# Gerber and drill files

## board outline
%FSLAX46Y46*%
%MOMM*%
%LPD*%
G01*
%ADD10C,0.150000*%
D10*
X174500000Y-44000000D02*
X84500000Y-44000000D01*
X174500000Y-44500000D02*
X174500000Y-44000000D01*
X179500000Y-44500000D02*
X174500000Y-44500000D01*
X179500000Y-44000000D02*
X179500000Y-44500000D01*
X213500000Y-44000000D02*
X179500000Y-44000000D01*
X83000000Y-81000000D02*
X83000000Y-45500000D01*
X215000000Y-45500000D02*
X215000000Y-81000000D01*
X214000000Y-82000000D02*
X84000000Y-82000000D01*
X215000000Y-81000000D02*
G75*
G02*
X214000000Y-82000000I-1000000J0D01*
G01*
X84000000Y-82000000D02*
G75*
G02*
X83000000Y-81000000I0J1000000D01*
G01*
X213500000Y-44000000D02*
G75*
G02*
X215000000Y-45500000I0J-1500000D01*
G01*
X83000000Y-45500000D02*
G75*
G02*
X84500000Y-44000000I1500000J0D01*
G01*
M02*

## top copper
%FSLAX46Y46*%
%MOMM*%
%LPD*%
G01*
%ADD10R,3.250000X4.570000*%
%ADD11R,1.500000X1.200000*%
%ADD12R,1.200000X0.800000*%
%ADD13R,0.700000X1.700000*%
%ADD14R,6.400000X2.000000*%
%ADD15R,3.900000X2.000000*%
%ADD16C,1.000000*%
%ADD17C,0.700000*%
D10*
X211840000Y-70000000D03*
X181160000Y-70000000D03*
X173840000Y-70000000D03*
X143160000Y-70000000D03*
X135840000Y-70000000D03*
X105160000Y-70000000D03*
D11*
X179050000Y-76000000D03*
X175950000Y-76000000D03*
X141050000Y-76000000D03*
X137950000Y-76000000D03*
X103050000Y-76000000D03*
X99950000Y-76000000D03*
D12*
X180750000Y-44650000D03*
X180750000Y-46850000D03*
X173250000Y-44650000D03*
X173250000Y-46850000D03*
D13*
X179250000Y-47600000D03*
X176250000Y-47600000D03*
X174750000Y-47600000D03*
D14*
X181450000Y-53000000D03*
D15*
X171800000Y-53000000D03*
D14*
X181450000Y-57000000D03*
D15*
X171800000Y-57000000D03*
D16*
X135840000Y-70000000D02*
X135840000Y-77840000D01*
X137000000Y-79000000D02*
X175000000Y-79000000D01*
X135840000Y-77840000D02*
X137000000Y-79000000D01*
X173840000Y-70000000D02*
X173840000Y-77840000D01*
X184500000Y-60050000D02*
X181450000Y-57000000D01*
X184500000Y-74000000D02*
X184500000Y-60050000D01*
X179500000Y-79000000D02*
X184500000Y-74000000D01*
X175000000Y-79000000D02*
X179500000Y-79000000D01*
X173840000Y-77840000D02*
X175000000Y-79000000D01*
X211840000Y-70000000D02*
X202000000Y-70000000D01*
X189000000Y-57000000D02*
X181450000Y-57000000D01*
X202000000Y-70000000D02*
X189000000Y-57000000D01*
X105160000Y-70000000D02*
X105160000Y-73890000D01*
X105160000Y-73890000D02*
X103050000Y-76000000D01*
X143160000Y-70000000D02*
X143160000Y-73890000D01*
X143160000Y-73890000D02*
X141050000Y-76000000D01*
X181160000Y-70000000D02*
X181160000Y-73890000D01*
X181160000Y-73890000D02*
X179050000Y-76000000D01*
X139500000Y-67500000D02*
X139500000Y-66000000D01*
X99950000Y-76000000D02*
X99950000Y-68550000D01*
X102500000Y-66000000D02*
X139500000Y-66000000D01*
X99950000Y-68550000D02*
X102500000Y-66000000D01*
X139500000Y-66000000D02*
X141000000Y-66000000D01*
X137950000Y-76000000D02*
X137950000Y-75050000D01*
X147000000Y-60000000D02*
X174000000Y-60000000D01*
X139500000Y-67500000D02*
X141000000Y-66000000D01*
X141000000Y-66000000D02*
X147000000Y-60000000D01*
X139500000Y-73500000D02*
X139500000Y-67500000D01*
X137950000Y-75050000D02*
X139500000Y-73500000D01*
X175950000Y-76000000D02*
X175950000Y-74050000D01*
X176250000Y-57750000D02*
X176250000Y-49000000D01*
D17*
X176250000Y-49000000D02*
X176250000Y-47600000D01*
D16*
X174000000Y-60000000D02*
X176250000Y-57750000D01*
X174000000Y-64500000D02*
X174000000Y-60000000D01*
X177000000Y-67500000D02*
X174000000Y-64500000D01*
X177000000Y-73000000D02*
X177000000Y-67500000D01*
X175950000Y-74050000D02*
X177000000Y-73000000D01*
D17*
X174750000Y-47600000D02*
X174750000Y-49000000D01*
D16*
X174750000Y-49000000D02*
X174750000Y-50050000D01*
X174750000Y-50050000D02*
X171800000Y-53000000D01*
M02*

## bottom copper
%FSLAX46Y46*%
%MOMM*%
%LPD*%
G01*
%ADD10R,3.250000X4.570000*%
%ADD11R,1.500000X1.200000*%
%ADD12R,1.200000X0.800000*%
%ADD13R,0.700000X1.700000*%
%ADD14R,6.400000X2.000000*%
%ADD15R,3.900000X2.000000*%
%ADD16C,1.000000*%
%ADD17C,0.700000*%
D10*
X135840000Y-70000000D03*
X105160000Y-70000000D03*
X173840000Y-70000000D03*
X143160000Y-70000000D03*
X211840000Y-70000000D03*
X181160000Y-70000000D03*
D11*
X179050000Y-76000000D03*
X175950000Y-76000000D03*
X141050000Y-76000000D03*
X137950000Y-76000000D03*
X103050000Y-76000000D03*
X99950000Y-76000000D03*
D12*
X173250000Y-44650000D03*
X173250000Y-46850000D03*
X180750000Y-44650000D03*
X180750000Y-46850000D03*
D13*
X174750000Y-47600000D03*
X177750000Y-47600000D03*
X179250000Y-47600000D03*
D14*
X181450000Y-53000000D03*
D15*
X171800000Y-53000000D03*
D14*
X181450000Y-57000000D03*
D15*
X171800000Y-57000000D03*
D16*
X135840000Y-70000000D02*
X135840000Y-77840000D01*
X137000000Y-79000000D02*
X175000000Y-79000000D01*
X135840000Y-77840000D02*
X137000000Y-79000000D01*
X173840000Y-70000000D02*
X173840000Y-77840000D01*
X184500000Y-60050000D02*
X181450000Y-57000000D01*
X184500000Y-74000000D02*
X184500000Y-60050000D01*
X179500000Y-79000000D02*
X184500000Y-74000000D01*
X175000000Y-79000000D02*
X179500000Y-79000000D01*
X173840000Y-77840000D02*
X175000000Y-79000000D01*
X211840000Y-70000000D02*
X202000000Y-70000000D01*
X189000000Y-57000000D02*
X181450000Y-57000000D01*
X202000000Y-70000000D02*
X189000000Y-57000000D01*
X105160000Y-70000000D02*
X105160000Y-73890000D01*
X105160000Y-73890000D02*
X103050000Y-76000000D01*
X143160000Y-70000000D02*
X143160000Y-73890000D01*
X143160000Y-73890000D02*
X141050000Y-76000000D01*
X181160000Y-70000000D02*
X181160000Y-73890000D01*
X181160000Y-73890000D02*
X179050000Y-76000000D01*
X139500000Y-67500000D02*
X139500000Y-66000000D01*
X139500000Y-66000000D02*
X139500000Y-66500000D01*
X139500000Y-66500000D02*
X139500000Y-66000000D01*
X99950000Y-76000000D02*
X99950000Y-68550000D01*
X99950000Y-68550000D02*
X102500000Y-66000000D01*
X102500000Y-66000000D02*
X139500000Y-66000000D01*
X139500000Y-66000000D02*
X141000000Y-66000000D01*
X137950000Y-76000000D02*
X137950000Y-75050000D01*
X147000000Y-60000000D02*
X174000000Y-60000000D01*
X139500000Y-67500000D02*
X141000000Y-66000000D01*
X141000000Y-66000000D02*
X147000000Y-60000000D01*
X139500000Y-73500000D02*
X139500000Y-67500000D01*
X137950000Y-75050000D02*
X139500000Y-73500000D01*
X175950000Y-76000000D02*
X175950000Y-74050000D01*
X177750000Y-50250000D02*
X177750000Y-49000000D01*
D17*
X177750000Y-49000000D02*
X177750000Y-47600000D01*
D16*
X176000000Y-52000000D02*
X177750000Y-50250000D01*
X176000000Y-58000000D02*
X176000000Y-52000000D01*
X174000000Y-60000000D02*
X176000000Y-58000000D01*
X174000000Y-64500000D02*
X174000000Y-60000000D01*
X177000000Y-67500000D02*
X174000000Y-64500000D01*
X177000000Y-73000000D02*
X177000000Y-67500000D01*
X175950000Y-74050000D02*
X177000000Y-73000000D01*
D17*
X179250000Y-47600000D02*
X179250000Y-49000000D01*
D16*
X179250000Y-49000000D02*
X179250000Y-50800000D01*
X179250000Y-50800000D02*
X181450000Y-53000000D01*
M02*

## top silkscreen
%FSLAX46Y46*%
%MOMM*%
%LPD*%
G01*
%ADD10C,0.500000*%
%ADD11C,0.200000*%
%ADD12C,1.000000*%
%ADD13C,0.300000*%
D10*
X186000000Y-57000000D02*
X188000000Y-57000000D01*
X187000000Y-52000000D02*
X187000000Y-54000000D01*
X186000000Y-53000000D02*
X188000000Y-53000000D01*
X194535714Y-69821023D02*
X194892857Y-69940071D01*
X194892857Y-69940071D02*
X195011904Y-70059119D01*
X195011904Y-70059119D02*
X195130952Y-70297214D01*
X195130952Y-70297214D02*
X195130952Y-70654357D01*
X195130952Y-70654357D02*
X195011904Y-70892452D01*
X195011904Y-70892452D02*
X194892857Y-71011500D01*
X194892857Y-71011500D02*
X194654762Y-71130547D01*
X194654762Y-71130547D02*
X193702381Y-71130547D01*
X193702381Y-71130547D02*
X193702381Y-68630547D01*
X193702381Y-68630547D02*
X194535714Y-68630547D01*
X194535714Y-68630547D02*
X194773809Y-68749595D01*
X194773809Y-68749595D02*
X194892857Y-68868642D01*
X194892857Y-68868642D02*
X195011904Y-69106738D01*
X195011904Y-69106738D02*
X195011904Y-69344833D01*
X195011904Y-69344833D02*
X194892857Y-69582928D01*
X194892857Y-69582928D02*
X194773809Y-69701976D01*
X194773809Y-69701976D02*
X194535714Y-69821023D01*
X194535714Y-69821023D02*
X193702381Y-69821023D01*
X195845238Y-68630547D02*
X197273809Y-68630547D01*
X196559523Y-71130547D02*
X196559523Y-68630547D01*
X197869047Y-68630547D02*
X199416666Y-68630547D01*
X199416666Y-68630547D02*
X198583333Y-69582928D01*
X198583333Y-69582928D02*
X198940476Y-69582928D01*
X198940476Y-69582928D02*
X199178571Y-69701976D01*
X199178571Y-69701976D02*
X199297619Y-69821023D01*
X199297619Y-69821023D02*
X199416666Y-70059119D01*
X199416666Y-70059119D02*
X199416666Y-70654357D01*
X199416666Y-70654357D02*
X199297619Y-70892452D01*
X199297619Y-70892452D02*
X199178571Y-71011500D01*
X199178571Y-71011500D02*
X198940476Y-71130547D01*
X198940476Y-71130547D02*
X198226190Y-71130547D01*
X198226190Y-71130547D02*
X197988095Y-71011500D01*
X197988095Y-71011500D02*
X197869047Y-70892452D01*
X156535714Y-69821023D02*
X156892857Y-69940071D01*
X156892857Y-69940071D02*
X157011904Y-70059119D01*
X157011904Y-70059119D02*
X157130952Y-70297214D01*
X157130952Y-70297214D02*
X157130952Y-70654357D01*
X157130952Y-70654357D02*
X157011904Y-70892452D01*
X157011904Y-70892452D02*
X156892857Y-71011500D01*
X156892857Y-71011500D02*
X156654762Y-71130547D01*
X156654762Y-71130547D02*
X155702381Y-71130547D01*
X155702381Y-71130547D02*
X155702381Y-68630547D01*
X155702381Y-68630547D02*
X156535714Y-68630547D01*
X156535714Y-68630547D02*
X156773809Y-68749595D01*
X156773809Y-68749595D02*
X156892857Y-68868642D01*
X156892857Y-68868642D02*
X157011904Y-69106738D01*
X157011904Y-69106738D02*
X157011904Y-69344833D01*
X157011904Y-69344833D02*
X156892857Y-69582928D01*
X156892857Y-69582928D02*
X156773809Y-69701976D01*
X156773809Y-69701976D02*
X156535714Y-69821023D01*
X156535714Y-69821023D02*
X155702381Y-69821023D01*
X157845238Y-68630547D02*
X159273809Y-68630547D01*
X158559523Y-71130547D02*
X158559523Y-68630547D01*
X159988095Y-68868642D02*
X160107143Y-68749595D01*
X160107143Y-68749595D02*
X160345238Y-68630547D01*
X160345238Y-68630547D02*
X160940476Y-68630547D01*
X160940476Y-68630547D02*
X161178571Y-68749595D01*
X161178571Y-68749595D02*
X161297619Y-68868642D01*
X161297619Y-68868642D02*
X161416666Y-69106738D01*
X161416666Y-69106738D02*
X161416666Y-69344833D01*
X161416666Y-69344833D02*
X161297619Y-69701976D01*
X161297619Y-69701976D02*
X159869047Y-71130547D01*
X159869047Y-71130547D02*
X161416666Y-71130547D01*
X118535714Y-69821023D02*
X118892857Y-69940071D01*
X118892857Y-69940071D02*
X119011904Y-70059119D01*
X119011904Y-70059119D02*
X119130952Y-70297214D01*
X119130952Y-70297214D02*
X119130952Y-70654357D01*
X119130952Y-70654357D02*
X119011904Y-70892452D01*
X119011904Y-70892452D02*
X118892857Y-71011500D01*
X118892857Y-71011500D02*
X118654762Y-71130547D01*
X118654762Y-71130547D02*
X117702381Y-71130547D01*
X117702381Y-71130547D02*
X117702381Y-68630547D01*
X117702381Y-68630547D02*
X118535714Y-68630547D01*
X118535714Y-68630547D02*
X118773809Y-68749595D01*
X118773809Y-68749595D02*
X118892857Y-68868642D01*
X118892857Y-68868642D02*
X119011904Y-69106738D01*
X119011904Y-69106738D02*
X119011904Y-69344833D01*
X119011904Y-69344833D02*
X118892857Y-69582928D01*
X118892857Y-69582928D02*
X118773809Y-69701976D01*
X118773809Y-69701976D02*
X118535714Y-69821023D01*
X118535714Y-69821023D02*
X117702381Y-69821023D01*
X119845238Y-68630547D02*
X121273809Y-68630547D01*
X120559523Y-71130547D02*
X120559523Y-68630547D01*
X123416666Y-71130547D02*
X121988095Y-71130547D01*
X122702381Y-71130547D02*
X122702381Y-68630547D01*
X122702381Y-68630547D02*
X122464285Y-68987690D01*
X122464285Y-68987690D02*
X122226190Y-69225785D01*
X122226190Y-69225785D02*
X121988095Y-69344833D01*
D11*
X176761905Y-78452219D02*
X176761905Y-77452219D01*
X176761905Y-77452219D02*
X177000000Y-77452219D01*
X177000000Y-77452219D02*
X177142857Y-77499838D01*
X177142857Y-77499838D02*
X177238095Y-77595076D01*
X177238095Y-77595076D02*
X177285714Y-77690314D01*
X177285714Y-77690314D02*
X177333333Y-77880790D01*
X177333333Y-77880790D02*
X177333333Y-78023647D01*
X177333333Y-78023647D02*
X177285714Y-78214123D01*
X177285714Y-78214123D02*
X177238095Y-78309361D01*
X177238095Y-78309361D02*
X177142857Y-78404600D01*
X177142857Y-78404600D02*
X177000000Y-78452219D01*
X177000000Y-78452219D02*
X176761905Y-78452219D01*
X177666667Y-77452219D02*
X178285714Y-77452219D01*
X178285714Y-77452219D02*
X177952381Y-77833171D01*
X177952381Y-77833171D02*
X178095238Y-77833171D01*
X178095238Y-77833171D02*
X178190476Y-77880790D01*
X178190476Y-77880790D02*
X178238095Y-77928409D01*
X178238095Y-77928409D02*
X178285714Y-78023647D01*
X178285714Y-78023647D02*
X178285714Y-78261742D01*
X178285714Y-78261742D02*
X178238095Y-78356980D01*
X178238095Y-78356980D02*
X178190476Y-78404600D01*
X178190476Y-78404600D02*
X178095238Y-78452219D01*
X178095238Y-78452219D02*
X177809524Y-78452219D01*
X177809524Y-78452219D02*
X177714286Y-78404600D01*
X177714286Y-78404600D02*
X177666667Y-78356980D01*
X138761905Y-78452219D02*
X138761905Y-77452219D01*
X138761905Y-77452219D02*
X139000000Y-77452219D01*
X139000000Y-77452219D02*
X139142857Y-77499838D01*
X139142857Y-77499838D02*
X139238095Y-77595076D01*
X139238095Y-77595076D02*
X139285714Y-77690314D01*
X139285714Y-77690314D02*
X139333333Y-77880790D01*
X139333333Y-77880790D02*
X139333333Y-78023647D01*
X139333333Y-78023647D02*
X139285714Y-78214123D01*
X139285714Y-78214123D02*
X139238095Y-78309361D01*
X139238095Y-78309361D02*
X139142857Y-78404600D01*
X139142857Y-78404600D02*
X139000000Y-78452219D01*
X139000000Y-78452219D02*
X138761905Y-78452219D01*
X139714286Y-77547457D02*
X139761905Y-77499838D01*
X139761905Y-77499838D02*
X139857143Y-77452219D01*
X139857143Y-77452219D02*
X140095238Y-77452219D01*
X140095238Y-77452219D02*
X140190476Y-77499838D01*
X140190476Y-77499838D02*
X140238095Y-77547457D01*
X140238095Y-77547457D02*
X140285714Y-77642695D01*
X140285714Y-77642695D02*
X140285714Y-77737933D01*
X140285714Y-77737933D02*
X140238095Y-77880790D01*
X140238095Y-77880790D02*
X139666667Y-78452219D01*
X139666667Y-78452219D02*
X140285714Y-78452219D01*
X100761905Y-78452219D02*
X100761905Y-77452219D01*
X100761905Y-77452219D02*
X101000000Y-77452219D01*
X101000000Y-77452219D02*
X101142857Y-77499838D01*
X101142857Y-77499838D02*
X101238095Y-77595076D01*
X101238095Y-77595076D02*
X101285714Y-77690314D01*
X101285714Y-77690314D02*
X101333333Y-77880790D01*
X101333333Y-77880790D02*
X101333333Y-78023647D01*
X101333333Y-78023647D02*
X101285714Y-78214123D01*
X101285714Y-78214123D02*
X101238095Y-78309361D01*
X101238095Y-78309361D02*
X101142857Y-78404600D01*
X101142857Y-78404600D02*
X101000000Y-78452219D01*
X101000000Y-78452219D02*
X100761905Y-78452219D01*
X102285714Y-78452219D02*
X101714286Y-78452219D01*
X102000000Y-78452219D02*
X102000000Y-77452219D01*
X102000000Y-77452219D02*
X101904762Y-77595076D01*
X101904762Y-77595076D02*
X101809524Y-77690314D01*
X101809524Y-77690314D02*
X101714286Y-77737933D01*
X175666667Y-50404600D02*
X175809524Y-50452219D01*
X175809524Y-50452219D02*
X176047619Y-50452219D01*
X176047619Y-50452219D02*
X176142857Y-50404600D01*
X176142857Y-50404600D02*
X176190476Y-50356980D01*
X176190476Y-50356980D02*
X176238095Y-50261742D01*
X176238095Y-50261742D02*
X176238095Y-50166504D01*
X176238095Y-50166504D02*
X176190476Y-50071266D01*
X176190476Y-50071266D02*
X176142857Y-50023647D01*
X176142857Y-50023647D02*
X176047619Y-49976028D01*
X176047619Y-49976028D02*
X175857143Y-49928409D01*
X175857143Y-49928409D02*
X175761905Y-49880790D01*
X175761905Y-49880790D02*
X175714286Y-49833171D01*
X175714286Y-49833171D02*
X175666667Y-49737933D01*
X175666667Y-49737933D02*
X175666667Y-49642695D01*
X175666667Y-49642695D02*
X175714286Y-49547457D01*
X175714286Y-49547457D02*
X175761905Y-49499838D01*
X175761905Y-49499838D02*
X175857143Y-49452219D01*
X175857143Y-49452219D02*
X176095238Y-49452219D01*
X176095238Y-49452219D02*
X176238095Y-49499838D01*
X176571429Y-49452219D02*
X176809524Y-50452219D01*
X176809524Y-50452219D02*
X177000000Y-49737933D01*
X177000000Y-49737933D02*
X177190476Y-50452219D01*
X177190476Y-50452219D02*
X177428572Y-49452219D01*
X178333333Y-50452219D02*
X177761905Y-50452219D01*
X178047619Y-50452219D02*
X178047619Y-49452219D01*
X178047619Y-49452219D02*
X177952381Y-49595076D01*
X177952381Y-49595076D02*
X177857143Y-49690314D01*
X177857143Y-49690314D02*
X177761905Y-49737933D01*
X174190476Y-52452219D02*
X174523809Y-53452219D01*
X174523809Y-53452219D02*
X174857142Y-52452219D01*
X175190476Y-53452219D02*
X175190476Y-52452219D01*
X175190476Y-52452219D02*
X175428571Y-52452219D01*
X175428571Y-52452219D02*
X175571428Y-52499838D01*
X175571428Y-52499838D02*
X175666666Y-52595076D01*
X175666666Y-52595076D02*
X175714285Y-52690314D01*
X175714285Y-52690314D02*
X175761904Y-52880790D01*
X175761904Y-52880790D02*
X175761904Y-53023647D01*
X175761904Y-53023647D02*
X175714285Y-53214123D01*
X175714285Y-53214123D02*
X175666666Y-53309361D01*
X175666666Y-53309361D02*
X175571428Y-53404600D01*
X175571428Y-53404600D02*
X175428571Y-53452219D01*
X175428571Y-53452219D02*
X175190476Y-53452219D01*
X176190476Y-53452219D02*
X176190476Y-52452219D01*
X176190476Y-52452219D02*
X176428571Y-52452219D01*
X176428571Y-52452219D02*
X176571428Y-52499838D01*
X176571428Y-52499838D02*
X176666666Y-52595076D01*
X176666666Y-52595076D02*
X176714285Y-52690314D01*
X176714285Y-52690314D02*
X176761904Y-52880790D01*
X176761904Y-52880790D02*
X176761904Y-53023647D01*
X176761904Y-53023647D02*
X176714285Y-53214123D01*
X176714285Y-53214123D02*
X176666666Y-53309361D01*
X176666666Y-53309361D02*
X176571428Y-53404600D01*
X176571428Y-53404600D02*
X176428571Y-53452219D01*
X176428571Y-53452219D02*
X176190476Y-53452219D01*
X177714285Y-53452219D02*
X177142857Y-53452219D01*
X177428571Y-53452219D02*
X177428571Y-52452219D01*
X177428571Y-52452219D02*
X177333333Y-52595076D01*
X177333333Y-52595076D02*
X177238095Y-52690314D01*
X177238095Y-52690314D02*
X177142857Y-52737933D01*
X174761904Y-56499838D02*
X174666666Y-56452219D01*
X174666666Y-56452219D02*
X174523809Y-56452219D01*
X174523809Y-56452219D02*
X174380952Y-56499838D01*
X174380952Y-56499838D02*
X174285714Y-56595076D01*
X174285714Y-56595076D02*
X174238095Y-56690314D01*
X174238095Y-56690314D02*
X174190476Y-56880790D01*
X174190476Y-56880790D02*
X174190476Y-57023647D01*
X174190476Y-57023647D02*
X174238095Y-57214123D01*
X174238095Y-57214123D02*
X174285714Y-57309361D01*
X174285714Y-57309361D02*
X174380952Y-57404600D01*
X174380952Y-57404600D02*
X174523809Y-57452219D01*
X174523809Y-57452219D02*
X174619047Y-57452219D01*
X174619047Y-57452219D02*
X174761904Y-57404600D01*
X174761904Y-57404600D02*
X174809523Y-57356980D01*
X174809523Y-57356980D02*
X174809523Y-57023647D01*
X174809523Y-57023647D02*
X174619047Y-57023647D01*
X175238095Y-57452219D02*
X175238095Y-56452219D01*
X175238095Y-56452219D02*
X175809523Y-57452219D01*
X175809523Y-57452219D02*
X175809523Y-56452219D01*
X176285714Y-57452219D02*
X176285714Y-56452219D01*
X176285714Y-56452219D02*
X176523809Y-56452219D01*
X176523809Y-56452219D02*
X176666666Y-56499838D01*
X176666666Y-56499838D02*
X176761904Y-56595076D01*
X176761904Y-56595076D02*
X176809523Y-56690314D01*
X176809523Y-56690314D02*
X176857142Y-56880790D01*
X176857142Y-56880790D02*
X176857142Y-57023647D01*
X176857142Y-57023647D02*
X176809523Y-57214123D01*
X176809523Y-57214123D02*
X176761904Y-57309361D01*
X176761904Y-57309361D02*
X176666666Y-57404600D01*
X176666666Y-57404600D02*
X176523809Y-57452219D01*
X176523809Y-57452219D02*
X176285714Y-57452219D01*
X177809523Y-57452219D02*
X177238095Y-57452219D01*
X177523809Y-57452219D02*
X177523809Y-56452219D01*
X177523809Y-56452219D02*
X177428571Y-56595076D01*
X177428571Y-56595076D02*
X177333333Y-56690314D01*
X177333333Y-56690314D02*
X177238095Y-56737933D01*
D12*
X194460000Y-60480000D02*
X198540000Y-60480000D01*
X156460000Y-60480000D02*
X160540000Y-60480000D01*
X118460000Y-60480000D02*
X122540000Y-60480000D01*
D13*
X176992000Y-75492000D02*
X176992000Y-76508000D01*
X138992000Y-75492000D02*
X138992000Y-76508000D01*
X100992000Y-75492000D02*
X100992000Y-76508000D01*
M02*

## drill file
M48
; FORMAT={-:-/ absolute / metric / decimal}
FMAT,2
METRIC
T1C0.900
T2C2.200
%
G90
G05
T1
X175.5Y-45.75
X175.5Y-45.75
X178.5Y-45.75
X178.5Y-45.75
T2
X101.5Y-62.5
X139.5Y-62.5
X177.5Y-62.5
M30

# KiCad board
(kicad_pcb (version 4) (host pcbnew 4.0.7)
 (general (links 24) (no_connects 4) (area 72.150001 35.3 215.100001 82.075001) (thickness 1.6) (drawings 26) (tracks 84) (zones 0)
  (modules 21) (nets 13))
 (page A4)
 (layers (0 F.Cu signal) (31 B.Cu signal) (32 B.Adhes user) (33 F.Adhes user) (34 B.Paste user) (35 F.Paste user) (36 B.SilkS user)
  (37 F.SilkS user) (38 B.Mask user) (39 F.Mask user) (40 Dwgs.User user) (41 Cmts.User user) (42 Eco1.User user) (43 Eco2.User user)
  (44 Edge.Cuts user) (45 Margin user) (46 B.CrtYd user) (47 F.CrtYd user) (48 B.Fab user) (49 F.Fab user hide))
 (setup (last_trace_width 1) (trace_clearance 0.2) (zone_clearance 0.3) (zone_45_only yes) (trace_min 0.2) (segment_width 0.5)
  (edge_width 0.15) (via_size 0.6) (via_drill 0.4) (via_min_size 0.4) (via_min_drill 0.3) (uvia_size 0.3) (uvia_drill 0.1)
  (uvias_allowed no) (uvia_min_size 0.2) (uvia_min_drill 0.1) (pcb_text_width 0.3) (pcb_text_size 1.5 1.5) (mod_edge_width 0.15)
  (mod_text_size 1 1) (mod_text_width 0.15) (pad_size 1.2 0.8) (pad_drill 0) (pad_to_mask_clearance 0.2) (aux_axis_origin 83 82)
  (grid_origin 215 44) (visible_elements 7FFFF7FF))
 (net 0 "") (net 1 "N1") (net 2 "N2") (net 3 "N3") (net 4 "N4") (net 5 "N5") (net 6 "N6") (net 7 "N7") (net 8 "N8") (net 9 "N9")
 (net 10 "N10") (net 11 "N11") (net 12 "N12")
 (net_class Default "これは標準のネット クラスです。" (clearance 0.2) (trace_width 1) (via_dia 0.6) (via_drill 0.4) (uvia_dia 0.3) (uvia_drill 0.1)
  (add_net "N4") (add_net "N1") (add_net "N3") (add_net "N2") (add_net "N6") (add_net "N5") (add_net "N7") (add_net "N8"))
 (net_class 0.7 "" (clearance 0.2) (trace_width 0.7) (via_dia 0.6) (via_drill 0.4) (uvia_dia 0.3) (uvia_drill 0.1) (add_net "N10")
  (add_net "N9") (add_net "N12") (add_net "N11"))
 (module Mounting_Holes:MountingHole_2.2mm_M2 (layer F.Cu) (at 101.5 62.5)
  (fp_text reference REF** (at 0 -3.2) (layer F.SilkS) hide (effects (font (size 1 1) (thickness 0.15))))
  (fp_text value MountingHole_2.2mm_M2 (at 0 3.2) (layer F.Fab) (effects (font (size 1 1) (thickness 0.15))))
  (pad 1 np_thru_hole circle (at 0 0) (size 2.2 2.2) (drill 2.2) (layers *.Cu *.Mask)))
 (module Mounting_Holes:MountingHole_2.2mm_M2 (layer F.Cu) (at 139.5 62.5)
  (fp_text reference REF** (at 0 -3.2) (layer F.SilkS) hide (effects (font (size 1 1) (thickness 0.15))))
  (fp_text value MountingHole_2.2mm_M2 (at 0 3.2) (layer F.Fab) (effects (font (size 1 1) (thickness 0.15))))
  (pad 1 np_thru_hole circle (at 0 0) (size 2.2 2.2) (drill 2.2) (layers *.Cu *.Mask)))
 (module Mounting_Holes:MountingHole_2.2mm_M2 (layer F.Cu) (at 177.5 62.5)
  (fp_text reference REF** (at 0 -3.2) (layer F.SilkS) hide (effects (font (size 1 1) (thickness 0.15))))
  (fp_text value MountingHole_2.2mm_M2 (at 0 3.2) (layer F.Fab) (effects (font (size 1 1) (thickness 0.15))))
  (pad 1 np_thru_hole circle (at 0 0) (size 2.2 2.2) (drill 2.2) (layers *.Cu *.Mask)))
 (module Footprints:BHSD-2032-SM (layer F.Cu) (at 196.5 70)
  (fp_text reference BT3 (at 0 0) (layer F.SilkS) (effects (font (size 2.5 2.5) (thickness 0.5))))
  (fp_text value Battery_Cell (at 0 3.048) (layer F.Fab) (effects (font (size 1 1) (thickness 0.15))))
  (fp_line (start -2.04 -9.52) (end 2.04 -9.52) (layer F.SilkS) (width 1))
  (pad 2 smd rect (at 15.34 0) (size 3.25 4.57) (layers F.Cu F.Paste F.Mask) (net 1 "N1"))
  (pad 1 smd rect (at -15.34 0) (size 3.25 4.57) (layers F.Cu F.Paste F.Mask) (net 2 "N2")))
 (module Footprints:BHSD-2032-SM (layer F.Cu) (at 158.5 70)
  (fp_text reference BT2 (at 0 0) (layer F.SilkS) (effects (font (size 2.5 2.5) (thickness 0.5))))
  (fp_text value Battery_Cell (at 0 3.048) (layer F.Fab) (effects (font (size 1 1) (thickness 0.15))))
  (fp_line (start -2.04 -9.52) (end 2.04 -9.52) (layer F.SilkS) (width 1))
  (pad 2 smd rect (at 15.34 0) (size 3.25 4.57) (layers F.Cu F.Paste F.Mask) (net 1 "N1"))
  (pad 1 smd rect (at -15.34 0) (size 3.25 4.57) (layers F.Cu F.Paste F.Mask) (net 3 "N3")))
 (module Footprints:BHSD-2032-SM (layer F.Cu) (at 120.5 70)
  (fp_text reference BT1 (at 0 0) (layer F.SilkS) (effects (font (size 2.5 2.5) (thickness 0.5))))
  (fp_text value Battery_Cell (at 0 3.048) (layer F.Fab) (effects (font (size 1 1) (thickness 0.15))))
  (fp_line (start -2.04 -9.52) (end 2.04 -9.52) (layer F.SilkS) (width 1))
  (pad 2 smd rect (at 15.34 0) (size 3.25 4.57) (layers F.Cu F.Paste F.Mask) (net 1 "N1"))
  (pad 1 smd rect (at -15.34 0) (size 3.25 4.57) (layers F.Cu F.Paste F.Mask) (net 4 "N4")))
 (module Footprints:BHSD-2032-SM (layer B.Cu) (at 120.5 70)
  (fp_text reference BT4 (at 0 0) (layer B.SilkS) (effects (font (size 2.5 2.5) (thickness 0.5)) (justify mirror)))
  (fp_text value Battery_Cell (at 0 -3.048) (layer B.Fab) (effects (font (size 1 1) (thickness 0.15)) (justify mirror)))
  (pad 2 smd rect (at 15.34 0) (size 3.25 4.57) (layers B.Cu B.Paste B.Mask) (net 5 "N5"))
  (pad 1 smd rect (at -15.34 0) (size 3.25 4.57) (layers B.Cu B.Paste B.Mask) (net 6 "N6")))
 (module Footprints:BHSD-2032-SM (layer B.Cu) (at 158.5 70)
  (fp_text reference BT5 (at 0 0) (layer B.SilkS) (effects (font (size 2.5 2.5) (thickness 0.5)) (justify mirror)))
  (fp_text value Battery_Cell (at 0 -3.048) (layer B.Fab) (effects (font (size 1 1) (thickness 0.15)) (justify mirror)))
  (pad 2 smd rect (at 15.34 0) (size 3.25 4.57) (layers B.Cu B.Paste B.Mask) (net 5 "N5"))
  (pad 1 smd rect (at -15.34 0) (size 3.25 4.57) (layers B.Cu B.Paste B.Mask) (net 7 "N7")))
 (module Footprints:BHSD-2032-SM (layer B.Cu) (at 196.5 70)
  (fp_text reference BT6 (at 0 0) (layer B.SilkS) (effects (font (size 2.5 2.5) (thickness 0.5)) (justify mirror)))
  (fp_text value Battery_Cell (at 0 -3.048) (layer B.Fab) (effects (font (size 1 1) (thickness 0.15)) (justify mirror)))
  (pad 2 smd rect (at 15.34 0) (size 3.25 4.57) (layers B.Cu B.Paste B.Mask) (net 5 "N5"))
  (pad 1 smd rect (at -15.34 0) (size 3.25 4.57) (layers B.Cu B.Paste B.Mask) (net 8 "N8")))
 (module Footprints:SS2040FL (layer B.Cu) (at 177.5 76)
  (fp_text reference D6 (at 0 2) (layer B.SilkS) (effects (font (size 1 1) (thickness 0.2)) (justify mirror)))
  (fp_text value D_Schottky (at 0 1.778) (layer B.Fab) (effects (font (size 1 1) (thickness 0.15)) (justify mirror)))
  (pad 2 smd rect (at 1.55 0) (size 1.5 1.2) (layers B.Cu B.Paste B.Mask) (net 8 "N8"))
  (pad 1 smd rect (at -1.55 0) (size 1.5 1.2) (layers B.Cu B.Paste B.Mask) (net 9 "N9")))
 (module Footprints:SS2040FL (layer B.Cu) (at 139.5 76)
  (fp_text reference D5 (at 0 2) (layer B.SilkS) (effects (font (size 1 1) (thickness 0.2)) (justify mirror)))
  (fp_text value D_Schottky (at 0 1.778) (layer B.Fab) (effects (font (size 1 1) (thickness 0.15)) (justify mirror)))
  (pad 2 smd rect (at 1.55 0) (size 1.5 1.2) (layers B.Cu B.Paste B.Mask) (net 7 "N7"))
  (pad 1 smd rect (at -1.55 0) (size 1.5 1.2) (layers B.Cu B.Paste B.Mask) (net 9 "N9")))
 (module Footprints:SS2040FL (layer B.Cu) (at 101.5 76)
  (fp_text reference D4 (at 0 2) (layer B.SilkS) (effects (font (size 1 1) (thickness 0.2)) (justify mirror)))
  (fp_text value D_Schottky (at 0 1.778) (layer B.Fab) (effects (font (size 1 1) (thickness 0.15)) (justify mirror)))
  (pad 2 smd rect (at 1.55 0) (size 1.5 1.2) (layers B.Cu B.Paste B.Mask) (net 6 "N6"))
  (pad 1 smd rect (at -1.55 0) (size 1.5 1.2) (layers B.Cu B.Paste B.Mask) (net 9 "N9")))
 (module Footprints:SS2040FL (layer F.Cu) (at 177.5 76)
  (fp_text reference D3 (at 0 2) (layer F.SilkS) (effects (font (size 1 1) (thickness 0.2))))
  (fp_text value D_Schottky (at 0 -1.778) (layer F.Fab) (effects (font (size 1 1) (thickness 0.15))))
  (fp_line (start -0.508 -0.508) (end -0.508 0.508) (layer F.SilkS) (width 0.3))
  (pad 2 smd rect (at 1.55 0) (size 1.5 1.2) (layers F.Cu F.Paste F.Mask) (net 2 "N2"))
  (pad 1 smd rect (at -1.55 0) (size 1.5 1.2) (layers F.Cu F.Paste F.Mask) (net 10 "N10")))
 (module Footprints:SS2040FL (layer F.Cu) (at 139.5 76)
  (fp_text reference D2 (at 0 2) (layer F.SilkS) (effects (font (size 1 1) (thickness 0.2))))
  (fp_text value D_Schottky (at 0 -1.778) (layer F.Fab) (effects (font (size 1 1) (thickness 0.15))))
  (fp_line (start -0.508 -0.508) (end -0.508 0.508) (layer F.SilkS) (width 0.3))
  (pad 2 smd rect (at 1.55 0) (size 1.5 1.2) (layers F.Cu F.Paste F.Mask) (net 3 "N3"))
  (pad 1 smd rect (at -1.55 0) (size 1.5 1.2) (layers F.Cu F.Paste F.Mask) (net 10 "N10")))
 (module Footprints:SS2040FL (layer F.Cu) (at 101.5 76)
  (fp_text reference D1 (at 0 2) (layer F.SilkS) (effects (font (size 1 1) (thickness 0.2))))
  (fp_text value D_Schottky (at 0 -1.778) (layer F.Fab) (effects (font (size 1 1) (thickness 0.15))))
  (fp_line (start -0.508 -0.508) (end -0.508 0.508) (layer F.SilkS) (width 0.3))
  (pad 2 smd rect (at 1.55 0) (size 1.5 1.2) (layers F.Cu F.Paste F.Mask) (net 4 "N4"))
  (pad 1 smd rect (at -1.55 0) (size 1.5 1.2) (layers F.Cu F.Paste F.Mask) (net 10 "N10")))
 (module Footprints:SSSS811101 (layer B.Cu) (at 177 45.75)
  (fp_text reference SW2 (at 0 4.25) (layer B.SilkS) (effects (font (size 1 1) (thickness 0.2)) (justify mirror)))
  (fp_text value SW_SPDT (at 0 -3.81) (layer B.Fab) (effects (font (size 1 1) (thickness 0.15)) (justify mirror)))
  (pad "" np_thru_hole circle (at -1.5 0) (size 0.9 0.9) (drill 0.9) (layers *.Cu *.Mask))
  (pad "" np_thru_hole circle (at 1.5 0) (size 0.9 0.9) (drill 0.9) (layers *.Cu *.Mask))
  (pad "" smd rect (at -3.75 -1.1) (size 1.2 0.8) (layers B.Cu B.Paste B.Mask))
  (pad "" smd rect (at -3.75 1.1) (size 1.2 0.8) (layers B.Cu B.Paste B.Mask))
  (pad "" smd rect (at 3.75 -1.1) (size 1.2 0.8) (layers B.Cu B.Paste B.Mask))
  (pad "" smd rect (at 3.75 1.1) (size 1.2 0.8) (layers B.Cu B.Paste B.Mask))
  (pad 1 smd rect (at -2.25 1.85) (size 0.7 1.7) (layers B.Cu B.Paste B.Mask))
  (pad 2 smd rect (at 0.75 1.85) (size 0.7 1.7) (layers B.Cu B.Paste B.Mask) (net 9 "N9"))
  (pad 3 smd rect (at 2.25 1.85) (size 0.7 1.7) (layers B.Cu B.Paste B.Mask) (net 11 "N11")))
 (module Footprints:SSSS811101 (layer F.Cu) (at 177 45.75 180)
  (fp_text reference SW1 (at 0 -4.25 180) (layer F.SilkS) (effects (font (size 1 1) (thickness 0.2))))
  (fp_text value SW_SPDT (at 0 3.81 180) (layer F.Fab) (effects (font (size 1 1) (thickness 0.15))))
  (pad "" np_thru_hole circle (at -1.5 0 180) (size 0.9 0.9) (drill 0.9) (layers *.Cu *.Mask))
  (pad "" np_thru_hole circle (at 1.5 0 180) (size 0.9 0.9) (drill 0.9) (layers *.Cu *.Mask))
  (pad "" smd rect (at -3.75 1.1 180) (size 1.2 0.8) (layers F.Cu F.Paste F.Mask))
  (pad "" smd rect (at -3.75 -1.1 180) (size 1.2 0.8) (layers F.Cu F.Paste F.Mask))
  (pad "" smd rect (at 3.75 1.1 180) (size 1.2 0.8) (layers F.Cu F.Paste F.Mask))
  (pad "" smd rect (at 3.75 -1.1 180) (size 1.2 0.8) (layers F.Cu F.Paste F.Mask))
  (pad 1 smd rect (at -2.25 -1.85 180) (size 0.7 1.7) (layers F.Cu F.Paste F.Mask))
  (pad 2 smd rect (at 0.75 -1.85 180) (size 0.7 1.7) (layers F.Cu F.Paste F.Mask) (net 10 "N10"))
  (pad 3 smd rect (at 2.25 -1.85 180) (size 0.7 1.7) (layers F.Cu F.Paste F.Mask) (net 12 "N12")))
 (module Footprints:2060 (layer B.Cu) (at 176 53 180)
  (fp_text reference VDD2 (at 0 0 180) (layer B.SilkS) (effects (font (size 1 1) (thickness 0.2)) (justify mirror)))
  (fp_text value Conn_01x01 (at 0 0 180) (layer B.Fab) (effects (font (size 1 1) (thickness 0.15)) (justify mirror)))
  (pad 1 smd rect (at -5.45 0 180) (size 6.4 2) (layers B.Cu B.Paste B.Mask) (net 11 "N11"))
  (pad 1 smd rect (at 4.2 0 180) (size 3.9 2) (layers B.Cu B.Paste B.Mask) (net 11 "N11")))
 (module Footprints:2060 (layer F.Cu) (at 176 53 180)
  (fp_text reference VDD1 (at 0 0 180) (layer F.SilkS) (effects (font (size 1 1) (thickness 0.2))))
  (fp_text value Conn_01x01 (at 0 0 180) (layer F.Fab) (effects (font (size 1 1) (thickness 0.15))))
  (pad 1 smd rect (at -5.45 0 180) (size 6.4 2) (layers F.Cu F.Paste F.Mask) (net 12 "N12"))
  (pad 1 smd rect (at 4.2 0 180) (size 3.9 2) (layers F.Cu F.Paste F.Mask) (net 12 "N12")))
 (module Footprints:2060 (layer B.Cu) (at 176 57 180)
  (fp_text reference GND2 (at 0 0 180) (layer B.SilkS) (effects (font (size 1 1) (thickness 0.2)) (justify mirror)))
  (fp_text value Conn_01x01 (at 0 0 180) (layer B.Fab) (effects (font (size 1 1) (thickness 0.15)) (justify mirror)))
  (pad 1 smd rect (at -5.45 0 180) (size 6.4 2) (layers B.Cu B.Paste B.Mask) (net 5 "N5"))
  (pad 1 smd rect (at 4.2 0 180) (size 3.9 2) (layers B.Cu B.Paste B.Mask) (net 5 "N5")))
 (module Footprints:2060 (layer F.Cu) (at 176 57 180)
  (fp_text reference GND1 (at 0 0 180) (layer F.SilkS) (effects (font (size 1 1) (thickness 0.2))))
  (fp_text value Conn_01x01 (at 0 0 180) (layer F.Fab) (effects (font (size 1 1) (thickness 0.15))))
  (pad 1 smd rect (at -5.45 0 180) (size 6.4 2) (layers F.Cu F.Paste F.Mask) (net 1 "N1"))
  (pad 1 smd rect (at 4.2 0 180) (size 3.9 2) (layers F.Cu F.Paste F.Mask) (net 1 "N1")))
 (gr_line (start 186 57) (end 188 57) (angle 90) (layer F.SilkS) (width 0.5))
 (gr_line (start 187 52) (end 187 54) (angle 90) (layer F.SilkS) (width 0.5))
 (gr_line (start 186 53) (end 188 53) (angle 90) (layer F.SilkS) (width 0.5))
 (gr_line (start 174.5 44) (end 84.5 44) (angle 90) (layer Edge.Cuts) (width 0.15))
 (gr_line (start 174.5 44.5) (end 174.5 44) (angle 90) (layer Edge.Cuts) (width 0.15))
 (gr_line (start 179.5 44.5) (end 174.5 44.5) (angle 90) (layer Edge.Cuts) (width 0.15))
 (gr_line (start 179.5 44) (end 179.5 44.5) (angle 90) (layer Edge.Cuts) (width 0.15))
 (gr_line (start 213.5 44) (end 179.5 44) (angle 90) (layer Edge.Cuts) (width 0.15))
 (gr_line (start 83 81) (end 83 45.5) (angle 90) (layer Edge.Cuts) (width 0.15))
 (gr_line (start 215 45.5) (end 215 81) (angle 90) (layer Edge.Cuts) (width 0.15))
 (gr_line (start 214 82) (end 84 82) (angle 90) (layer Edge.Cuts) (width 0.15))
 (gr_arc (start 214 81) (end 215 81) (angle 90) (layer Edge.Cuts) (width 0.15))
 (gr_arc (start 84 81) (end 84 82) (angle 90) (layer Edge.Cuts) (width 0.15))
 (gr_arc (start 213.5 45.5) (end 213.5 44) (angle 90) (layer Edge.Cuts) (width 0.15))
 (gr_arc (start 84.5 45.5) (end 83 45.5) (angle 90) (layer Edge.Cuts) (width 0.15))
 (segment (start 135.84 70) (end 135.84 77.84) (width 1) (layer F.Cu) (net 1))
 (segment (start 137 79) (end 175 79) (width 1) (layer F.Cu) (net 1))
 (segment (start 135.84 77.84) (end 137 79) (width 1) (layer F.Cu) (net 1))
 (segment (start 173.84 70) (end 173.84 77.84) (width 1) (layer F.Cu) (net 1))
 (segment (start 184.5 60.05) (end 181.45 57) (width 1) (layer F.Cu) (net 1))
 (segment (start 184.5 74) (end 184.5 60.05) (width 1) (layer F.Cu) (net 1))
 (segment (start 179.5 79) (end 184.5 74) (width 1) (layer F.Cu) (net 1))
 (segment (start 175 79) (end 179.5 79) (width 1) (layer F.Cu) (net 1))
 (segment (start 173.84 77.84) (end 175 79) (width 1) (layer F.Cu) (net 1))
 (segment (start 211.84 70) (end 202 70) (width 1) (layer F.Cu) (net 1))
 (segment (start 189 57) (end 181.45 57) (width 1) (layer F.Cu) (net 1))
 (segment (start 202 70) (end 189 57) (width 1) (layer F.Cu) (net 1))
 (segment (start 105.16 70) (end 105.16 73.89) (width 1) (layer F.Cu) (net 4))
 (segment (start 105.16 73.89) (end 103.05 76) (width 1) (layer F.Cu) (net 4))
 (segment (start 143.16 70) (end 143.16 73.89) (width 1) (layer F.Cu) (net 3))
 (segment (start 143.16 73.89) (end 141.05 76) (width 1) (layer F.Cu) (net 3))
 (segment (start 181.16 70) (end 181.16 73.89) (width 1) (layer F.Cu) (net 2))
 (segment (start 181.16 73.89) (end 179.05 76) (width 1) (layer F.Cu) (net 2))
 (segment (start 139.5 67.5) (end 139.5 66) (width 1) (layer F.Cu) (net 10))
 (segment (start 99.95 76) (end 99.95 68.55) (width 1) (layer F.Cu) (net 10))
 (segment (start 102.5 66) (end 139.5 66) (width 1) (layer F.Cu) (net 10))
 (segment (start 99.95 68.55) (end 102.5 66) (width 1) (layer F.Cu) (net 10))
 (segment (start 139.5 66) (end 141 66) (width 1) (layer F.Cu) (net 10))
 (segment (start 137.95 76) (end 137.95 75.05) (width 1) (layer F.Cu) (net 10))
 (segment (start 147 60) (end 174 60) (width 1) (layer F.Cu) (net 10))
 (segment (start 139.5 67.5) (end 141 66) (width 1) (layer F.Cu) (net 10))
 (segment (start 141 66) (end 147 60) (width 1) (layer F.Cu) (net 10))
 (segment (start 139.5 73.5) (end 139.5 67.5) (width 1) (layer F.Cu) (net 10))
 (segment (start 137.95 75.05) (end 139.5 73.5) (width 1) (layer F.Cu) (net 10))
 (segment (start 175.95 76) (end 175.95 74.05) (width 1) (layer F.Cu) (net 10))
 (segment (start 176.25 57.75) (end 176.25 49) (width 1) (layer F.Cu) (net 10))
 (segment (start 176.25 49) (end 176.25 47.6) (width 0.7) (layer F.Cu) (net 10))
 (segment (start 174 60) (end 176.25 57.75) (width 1) (layer F.Cu) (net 10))
 (segment (start 174 64.5) (end 174 60) (width 1) (layer F.Cu) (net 10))
 (segment (start 177 67.5) (end 174 64.5) (width 1) (layer F.Cu) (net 10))
 (segment (start 177 73) (end 177 67.5) (width 1) (layer F.Cu) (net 10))
 (segment (start 175.95 74.05) (end 177 73) (width 1) (layer F.Cu) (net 10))
 (segment (start 135.84 70) (end 135.84 77.84) (width 1) (layer B.Cu) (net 5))
 (segment (start 137 79) (end 175 79) (width 1) (layer B.Cu) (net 5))
 (segment (start 135.84 77.84) (end 137 79) (width 1) (layer B.Cu) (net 5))
 (segment (start 173.84 70) (end 173.84 77.84) (width 1) (layer B.Cu) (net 5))
 (segment (start 184.5 60.05) (end 181.45 57) (width 1) (layer B.Cu) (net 5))
 (segment (start 184.5 74) (end 184.5 60.05) (width 1) (layer B.Cu) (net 5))
 (segment (start 179.5 79) (end 184.5 74) (width 1) (layer B.Cu) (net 5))
 (segment (start 175 79) (end 179.5 79) (width 1) (layer B.Cu) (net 5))
 (segment (start 173.84 77.84) (end 175 79) (width 1) (layer B.Cu) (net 5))
 (segment (start 211.84 70) (end 202 70) (width 1) (layer B.Cu) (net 5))
 (segment (start 189 57) (end 181.45 57) (width 1) (layer B.Cu) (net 5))
 (segment (start 202 70) (end 189 57) (width 1) (layer B.Cu) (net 5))
 (segment (start 105.16 70) (end 105.16 73.89) (width 1) (layer B.Cu) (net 6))
 (segment (start 105.16 73.89) (end 103.05 76) (width 1) (layer B.Cu) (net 6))
 (segment (start 143.16 70) (end 143.16 73.89) (width 1) (layer B.Cu) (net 7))
 (segment (start 143.16 73.89) (end 141.05 76) (width 1) (layer B.Cu) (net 7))
 (segment (start 181.16 70) (end 181.16 73.89) (width 1) (layer B.Cu) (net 8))
 (segment (start 181.16 73.89) (end 179.05 76) (width 1) (layer B.Cu) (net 8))
 (segment (start 139.5 67.5) (end 139.5 66) (width 1) (layer B.Cu) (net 9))
 (segment (start 139.5 66) (end 139.5 66.5) (width 1) (layer B.Cu) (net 9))
 (segment (start 139.5 66.5) (end 139.5 66) (width 1) (layer B.Cu) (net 9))
 (segment (start 99.95 76) (end 99.95 68.55) (width 1) (layer B.Cu) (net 9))
 (segment (start 99.95 68.55) (end 102.5 66) (width 1) (layer B.Cu) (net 9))
 (segment (start 102.5 66) (end 139.5 66) (width 1) (layer B.Cu) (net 9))
 (segment (start 139.5 66) (end 141 66) (width 1) (layer B.Cu) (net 9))
 (segment (start 137.95 76) (end 137.95 75.05) (width 1) (layer B.Cu) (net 9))
 (segment (start 147 60) (end 174 60) (width 1) (layer B.Cu) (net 9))
 (segment (start 139.5 67.5) (end 141 66) (width 1) (layer B.Cu) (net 9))
 (segment (start 141 66) (end 147 60) (width 1) (layer B.Cu) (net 9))
 (segment (start 139.5 73.5) (end 139.5 67.5) (width 1) (layer B.Cu) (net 9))
 (segment (start 137.95 75.05) (end 139.5 73.5) (width 1) (layer B.Cu) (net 9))
 (segment (start 175.95 76) (end 175.95 74.05) (width 1) (layer B.Cu) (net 9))
 (segment (start 177.75 50.25) (end 177.75 49) (width 1) (layer B.Cu) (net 9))
 (segment (start 177.75 49) (end 177.75 47.6) (width 0.7) (layer B.Cu) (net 9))
 (segment (start 176 52) (end 177.75 50.25) (width 1) (layer B.Cu) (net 9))
 (segment (start 176 58) (end 176 52) (width 1) (layer B.Cu) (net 9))
 (segment (start 174 60) (end 176 58) (width 1) (layer B.Cu) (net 9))
 (segment (start 174 64.5) (end 174 60) (width 1) (layer B.Cu) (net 9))
 (segment (start 177 67.5) (end 174 64.5) (width 1) (layer B.Cu) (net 9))
 (segment (start 177 73) (end 177 67.5) (width 1) (layer B.Cu) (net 9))
 (segment (start 175.95 74.05) (end 177 73) (width 1) (layer B.Cu) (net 9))
 (segment (start 174.75 47.6) (end 174.75 49) (width 0.7) (layer F.Cu) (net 12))
 (segment (start 174.75 49) (end 174.75 50.05) (width 1) (layer F.Cu) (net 12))
 (segment (start 174.75 50.05) (end 171.8 53) (width 1) (layer F.Cu) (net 12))
 (segment (start 179.25 47.6) (end 179.25 49) (width 0.7) (layer B.Cu) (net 11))
 (segment (start 179.25 49) (end 179.25 50.8) (width 1) (layer B.Cu) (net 11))
 (segment (start 179.25 50.8) (end 181.45 53) (width 1) (layer B.Cu) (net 11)))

